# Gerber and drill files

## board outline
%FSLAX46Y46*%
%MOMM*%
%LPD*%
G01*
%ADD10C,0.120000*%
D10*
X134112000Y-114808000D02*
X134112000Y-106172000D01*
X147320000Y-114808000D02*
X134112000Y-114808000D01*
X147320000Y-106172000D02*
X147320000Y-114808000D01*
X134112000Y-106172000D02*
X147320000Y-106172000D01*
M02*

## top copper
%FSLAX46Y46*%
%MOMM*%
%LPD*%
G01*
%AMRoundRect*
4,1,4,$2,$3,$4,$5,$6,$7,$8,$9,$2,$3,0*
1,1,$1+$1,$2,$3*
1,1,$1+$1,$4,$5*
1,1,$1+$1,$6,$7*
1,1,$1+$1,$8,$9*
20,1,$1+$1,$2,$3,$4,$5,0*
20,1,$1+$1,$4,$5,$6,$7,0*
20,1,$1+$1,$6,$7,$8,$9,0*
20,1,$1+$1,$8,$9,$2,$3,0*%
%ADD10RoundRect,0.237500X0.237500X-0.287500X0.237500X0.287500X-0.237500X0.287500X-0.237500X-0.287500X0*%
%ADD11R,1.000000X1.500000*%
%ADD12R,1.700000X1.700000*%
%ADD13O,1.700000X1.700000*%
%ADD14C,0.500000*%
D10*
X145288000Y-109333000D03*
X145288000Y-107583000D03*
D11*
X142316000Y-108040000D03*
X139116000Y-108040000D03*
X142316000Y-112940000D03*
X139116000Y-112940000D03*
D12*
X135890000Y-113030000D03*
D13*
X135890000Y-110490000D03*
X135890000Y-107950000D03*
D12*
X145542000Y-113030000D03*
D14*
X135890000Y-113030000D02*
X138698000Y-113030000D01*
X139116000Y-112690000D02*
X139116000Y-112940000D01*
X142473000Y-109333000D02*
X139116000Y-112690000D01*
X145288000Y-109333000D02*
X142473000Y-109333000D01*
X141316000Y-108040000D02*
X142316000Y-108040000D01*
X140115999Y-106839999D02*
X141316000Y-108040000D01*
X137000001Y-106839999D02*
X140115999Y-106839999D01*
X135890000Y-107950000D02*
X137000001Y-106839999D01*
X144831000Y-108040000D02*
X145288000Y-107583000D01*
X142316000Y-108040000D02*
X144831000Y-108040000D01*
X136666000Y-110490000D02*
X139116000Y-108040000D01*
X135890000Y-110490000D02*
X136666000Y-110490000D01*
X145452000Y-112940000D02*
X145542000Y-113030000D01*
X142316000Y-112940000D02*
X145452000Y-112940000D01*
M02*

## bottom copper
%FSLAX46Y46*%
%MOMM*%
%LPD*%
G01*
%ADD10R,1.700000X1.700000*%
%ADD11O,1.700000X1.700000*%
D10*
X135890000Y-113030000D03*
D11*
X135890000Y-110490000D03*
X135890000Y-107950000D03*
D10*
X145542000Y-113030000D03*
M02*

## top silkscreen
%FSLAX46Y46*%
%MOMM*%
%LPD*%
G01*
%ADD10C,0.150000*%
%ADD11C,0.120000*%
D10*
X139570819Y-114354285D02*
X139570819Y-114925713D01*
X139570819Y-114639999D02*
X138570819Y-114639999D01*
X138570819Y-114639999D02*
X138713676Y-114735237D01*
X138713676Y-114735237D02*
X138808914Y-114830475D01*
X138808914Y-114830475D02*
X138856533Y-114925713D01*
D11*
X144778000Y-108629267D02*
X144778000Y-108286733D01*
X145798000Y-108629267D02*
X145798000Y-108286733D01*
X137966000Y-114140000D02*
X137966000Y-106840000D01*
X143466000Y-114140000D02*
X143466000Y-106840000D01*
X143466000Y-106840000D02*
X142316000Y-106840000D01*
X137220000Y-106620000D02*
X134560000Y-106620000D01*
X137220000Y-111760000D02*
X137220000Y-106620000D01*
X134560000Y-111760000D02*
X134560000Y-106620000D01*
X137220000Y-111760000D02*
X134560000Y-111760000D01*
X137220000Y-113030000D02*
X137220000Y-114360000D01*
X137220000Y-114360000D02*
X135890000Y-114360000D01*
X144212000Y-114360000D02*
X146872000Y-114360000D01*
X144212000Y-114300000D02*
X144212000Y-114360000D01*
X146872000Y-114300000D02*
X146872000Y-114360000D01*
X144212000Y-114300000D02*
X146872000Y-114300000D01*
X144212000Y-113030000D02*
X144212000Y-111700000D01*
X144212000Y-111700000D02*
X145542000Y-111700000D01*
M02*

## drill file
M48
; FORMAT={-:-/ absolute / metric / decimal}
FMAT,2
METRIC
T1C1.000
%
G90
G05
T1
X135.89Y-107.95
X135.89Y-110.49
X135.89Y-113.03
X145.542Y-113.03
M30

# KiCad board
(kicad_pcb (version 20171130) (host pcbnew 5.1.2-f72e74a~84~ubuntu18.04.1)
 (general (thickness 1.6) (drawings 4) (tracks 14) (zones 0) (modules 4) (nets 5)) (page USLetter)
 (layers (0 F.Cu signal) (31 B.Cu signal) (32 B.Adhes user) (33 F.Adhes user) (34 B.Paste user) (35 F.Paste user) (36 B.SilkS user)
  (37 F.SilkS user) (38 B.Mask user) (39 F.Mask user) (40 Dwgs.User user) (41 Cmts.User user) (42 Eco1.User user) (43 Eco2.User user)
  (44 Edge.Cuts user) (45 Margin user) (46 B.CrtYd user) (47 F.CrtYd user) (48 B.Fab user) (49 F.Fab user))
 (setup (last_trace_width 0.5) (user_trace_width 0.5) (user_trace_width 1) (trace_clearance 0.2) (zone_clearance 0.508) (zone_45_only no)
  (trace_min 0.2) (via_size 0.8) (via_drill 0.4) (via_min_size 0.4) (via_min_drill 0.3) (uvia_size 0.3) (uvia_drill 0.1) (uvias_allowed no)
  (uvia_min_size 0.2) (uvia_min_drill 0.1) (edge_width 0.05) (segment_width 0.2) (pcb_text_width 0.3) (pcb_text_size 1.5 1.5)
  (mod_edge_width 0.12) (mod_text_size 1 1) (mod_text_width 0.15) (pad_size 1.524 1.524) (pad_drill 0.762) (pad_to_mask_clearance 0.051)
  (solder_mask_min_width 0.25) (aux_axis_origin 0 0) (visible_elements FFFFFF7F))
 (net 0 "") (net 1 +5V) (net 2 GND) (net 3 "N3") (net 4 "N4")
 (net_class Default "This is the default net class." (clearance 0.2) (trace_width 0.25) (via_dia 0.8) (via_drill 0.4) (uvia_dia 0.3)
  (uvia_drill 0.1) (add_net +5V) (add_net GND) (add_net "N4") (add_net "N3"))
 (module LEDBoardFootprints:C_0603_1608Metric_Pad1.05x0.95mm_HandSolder (layer F.Cu) (at 145.288 108.458 90)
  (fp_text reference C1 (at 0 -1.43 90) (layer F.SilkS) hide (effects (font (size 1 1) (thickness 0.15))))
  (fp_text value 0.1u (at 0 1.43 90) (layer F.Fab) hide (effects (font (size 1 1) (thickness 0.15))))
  (fp_line (start -0.171267 -0.51) (end 0.171267 -0.51) (layer F.SilkS) (width 0.12))
  (fp_line (start -0.171267 0.51) (end 0.171267 0.51) (layer F.SilkS) (width 0.12))
  (pad 1 smd roundrect (at -0.875 0 90) (size 1.05 0.95) (layers F.Cu F.Paste F.Mask) (roundrect_rratio 0.25) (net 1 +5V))
  (pad 2 smd roundrect (at 0.875 0 90) (size 1.05 0.95) (layers F.Cu F.Paste F.Mask) (roundrect_rratio 0.25) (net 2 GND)))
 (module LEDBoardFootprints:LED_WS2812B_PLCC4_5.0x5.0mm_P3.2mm (layer F.Cu) (at 140.716 110.49 90)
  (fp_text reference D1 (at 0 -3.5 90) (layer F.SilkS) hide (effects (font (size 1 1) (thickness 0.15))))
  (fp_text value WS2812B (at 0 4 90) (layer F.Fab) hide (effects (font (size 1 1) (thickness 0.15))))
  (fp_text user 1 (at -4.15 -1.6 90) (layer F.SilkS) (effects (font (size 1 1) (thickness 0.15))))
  (fp_line (start -3.65 -2.75) (end 3.65 -2.75) (layer F.SilkS) (width 0.12))
  (fp_line (start -3.65 2.75) (end 3.65 2.75) (layer F.SilkS) (width 0.12))
  (fp_line (start 3.65 2.75) (end 3.65 1.6) (layer F.SilkS) (width 0.12))
  (pad 3 smd rect (at 2.45 1.6 90) (size 1.5 1) (layers F.Cu F.Paste F.Mask) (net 2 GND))
  (pad 4 smd rect (at 2.45 -1.6 90) (size 1.5 1) (layers F.Cu F.Paste F.Mask) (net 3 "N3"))
  (pad 2 smd rect (at -2.45 1.6 90) (size 1.5 1) (layers F.Cu F.Paste F.Mask) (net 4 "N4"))
  (pad 1 smd rect (at -2.45 -1.6 90) (size 1.5 1) (layers F.Cu F.Paste F.Mask) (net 1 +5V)))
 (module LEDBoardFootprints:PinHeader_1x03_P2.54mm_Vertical (layer F.Cu) (at 135.89 113.03 180)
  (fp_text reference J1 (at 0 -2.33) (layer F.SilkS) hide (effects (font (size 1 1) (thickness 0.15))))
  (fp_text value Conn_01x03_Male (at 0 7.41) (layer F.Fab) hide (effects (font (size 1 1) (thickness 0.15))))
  (fp_line (start -1.33 6.41) (end 1.33 6.41) (layer F.SilkS) (width 0.12))
  (fp_line (start -1.33 1.27) (end -1.33 6.41) (layer F.SilkS) (width 0.12))
  (fp_line (start 1.33 1.27) (end 1.33 6.41) (layer F.SilkS) (width 0.12))
  (fp_line (start -1.33 1.27) (end 1.33 1.27) (layer F.SilkS) (width 0.12))
  (fp_line (start -1.33 0) (end -1.33 -1.33) (layer F.SilkS) (width 0.12))
  (fp_line (start -1.33 -1.33) (end 0 -1.33) (layer F.SilkS) (width 0.12))
  (pad 1 thru_hole rect (at 0 0 180) (size 1.7 1.7) (drill 1) (layers *.Cu *.Mask) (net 1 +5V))
  (pad 2 thru_hole oval (at 0 2.54 180) (size 1.7 1.7) (drill 1) (layers *.Cu *.Mask) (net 3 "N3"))
  (pad 3 thru_hole oval (at 0 5.08 180) (size 1.7 1.7) (drill 1) (layers *.Cu *.Mask) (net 2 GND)))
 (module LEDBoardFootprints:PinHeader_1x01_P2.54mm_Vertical (layer F.Cu) (at 145.542 113.03)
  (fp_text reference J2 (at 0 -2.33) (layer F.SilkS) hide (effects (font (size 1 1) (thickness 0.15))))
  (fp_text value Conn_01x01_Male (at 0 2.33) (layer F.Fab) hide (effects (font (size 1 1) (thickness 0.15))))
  (fp_line (start -1.33 1.33) (end 1.33 1.33) (layer F.SilkS) (width 0.12))
  (fp_line (start -1.33 1.27) (end -1.33 1.33) (layer F.SilkS) (width 0.12))
  (fp_line (start 1.33 1.27) (end 1.33 1.33) (layer F.SilkS) (width 0.12))
  (fp_line (start -1.33 1.27) (end 1.33 1.27) (layer F.SilkS) (width 0.12))
  (fp_line (start -1.33 0) (end -1.33 -1.33) (layer F.SilkS) (width 0.12))
  (fp_line (start -1.33 -1.33) (end 0 -1.33) (layer F.SilkS) (width 0.12))
  (pad 1 thru_hole rect (at 0 0) (size 1.7 1.7) (drill 1) (layers *.Cu *.Mask) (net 4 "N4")))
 (gr_line (start 134.112 114.808) (end 134.112 106.172) (layer Edge.Cuts) (width 0.12))
 (gr_line (start 147.32 114.808) (end 134.112 114.808) (layer Edge.Cuts) (width 0.12))
 (gr_line (start 147.32 106.172) (end 147.32 114.808) (layer Edge.Cuts) (width 0.12))
 (gr_line (start 134.112 106.172) (end 147.32 106.172) (layer Edge.Cuts) (width 0.12))
 (segment (start 135.89 113.03) (end 138.698 113.03) (width 0.5) (layer F.Cu) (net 1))
 (segment (start 139.116 112.69) (end 139.116 112.94) (width 0.5) (layer F.Cu) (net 1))
 (segment (start 142.473 109.333) (end 139.116 112.69) (width 0.5) (layer F.Cu) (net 1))
 (segment (start 145.288 109.333) (end 142.473 109.333) (width 0.5) (layer F.Cu) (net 1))
 (segment (start 141.316 108.04) (end 142.316 108.04) (width 0.5) (layer F.Cu) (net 2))
 (segment (start 140.115999 106.839999) (end 141.316 108.04) (width 0.5) (layer F.Cu) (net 2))
 (segment (start 137.000001 106.839999) (end 140.115999 106.839999) (width 0.5) (layer F.Cu) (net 2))
 (segment (start 135.89 107.95) (end 137.000001 106.839999) (width 0.5) (layer F.Cu) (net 2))
 (segment (start 144.831 108.04) (end 145.288 107.583) (width 0.5) (layer F.Cu) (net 2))
 (segment (start 142.316 108.04) (end 144.831 108.04) (width 0.5) (layer F.Cu) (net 2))
 (segment (start 136.666 110.49) (end 139.116 108.04) (width 0.5) (layer F.Cu) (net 3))
 (segment (start 135.89 110.49) (end 136.666 110.49) (width 0.5) (layer F.Cu) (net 3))
 (segment (start 145.452 112.94) (end 145.542 113.03) (width 0.5) (layer F.Cu) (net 4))
 (segment (start 142.316 112.94) (end 145.452 112.94) (width 0.5) (layer F.Cu) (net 4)))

